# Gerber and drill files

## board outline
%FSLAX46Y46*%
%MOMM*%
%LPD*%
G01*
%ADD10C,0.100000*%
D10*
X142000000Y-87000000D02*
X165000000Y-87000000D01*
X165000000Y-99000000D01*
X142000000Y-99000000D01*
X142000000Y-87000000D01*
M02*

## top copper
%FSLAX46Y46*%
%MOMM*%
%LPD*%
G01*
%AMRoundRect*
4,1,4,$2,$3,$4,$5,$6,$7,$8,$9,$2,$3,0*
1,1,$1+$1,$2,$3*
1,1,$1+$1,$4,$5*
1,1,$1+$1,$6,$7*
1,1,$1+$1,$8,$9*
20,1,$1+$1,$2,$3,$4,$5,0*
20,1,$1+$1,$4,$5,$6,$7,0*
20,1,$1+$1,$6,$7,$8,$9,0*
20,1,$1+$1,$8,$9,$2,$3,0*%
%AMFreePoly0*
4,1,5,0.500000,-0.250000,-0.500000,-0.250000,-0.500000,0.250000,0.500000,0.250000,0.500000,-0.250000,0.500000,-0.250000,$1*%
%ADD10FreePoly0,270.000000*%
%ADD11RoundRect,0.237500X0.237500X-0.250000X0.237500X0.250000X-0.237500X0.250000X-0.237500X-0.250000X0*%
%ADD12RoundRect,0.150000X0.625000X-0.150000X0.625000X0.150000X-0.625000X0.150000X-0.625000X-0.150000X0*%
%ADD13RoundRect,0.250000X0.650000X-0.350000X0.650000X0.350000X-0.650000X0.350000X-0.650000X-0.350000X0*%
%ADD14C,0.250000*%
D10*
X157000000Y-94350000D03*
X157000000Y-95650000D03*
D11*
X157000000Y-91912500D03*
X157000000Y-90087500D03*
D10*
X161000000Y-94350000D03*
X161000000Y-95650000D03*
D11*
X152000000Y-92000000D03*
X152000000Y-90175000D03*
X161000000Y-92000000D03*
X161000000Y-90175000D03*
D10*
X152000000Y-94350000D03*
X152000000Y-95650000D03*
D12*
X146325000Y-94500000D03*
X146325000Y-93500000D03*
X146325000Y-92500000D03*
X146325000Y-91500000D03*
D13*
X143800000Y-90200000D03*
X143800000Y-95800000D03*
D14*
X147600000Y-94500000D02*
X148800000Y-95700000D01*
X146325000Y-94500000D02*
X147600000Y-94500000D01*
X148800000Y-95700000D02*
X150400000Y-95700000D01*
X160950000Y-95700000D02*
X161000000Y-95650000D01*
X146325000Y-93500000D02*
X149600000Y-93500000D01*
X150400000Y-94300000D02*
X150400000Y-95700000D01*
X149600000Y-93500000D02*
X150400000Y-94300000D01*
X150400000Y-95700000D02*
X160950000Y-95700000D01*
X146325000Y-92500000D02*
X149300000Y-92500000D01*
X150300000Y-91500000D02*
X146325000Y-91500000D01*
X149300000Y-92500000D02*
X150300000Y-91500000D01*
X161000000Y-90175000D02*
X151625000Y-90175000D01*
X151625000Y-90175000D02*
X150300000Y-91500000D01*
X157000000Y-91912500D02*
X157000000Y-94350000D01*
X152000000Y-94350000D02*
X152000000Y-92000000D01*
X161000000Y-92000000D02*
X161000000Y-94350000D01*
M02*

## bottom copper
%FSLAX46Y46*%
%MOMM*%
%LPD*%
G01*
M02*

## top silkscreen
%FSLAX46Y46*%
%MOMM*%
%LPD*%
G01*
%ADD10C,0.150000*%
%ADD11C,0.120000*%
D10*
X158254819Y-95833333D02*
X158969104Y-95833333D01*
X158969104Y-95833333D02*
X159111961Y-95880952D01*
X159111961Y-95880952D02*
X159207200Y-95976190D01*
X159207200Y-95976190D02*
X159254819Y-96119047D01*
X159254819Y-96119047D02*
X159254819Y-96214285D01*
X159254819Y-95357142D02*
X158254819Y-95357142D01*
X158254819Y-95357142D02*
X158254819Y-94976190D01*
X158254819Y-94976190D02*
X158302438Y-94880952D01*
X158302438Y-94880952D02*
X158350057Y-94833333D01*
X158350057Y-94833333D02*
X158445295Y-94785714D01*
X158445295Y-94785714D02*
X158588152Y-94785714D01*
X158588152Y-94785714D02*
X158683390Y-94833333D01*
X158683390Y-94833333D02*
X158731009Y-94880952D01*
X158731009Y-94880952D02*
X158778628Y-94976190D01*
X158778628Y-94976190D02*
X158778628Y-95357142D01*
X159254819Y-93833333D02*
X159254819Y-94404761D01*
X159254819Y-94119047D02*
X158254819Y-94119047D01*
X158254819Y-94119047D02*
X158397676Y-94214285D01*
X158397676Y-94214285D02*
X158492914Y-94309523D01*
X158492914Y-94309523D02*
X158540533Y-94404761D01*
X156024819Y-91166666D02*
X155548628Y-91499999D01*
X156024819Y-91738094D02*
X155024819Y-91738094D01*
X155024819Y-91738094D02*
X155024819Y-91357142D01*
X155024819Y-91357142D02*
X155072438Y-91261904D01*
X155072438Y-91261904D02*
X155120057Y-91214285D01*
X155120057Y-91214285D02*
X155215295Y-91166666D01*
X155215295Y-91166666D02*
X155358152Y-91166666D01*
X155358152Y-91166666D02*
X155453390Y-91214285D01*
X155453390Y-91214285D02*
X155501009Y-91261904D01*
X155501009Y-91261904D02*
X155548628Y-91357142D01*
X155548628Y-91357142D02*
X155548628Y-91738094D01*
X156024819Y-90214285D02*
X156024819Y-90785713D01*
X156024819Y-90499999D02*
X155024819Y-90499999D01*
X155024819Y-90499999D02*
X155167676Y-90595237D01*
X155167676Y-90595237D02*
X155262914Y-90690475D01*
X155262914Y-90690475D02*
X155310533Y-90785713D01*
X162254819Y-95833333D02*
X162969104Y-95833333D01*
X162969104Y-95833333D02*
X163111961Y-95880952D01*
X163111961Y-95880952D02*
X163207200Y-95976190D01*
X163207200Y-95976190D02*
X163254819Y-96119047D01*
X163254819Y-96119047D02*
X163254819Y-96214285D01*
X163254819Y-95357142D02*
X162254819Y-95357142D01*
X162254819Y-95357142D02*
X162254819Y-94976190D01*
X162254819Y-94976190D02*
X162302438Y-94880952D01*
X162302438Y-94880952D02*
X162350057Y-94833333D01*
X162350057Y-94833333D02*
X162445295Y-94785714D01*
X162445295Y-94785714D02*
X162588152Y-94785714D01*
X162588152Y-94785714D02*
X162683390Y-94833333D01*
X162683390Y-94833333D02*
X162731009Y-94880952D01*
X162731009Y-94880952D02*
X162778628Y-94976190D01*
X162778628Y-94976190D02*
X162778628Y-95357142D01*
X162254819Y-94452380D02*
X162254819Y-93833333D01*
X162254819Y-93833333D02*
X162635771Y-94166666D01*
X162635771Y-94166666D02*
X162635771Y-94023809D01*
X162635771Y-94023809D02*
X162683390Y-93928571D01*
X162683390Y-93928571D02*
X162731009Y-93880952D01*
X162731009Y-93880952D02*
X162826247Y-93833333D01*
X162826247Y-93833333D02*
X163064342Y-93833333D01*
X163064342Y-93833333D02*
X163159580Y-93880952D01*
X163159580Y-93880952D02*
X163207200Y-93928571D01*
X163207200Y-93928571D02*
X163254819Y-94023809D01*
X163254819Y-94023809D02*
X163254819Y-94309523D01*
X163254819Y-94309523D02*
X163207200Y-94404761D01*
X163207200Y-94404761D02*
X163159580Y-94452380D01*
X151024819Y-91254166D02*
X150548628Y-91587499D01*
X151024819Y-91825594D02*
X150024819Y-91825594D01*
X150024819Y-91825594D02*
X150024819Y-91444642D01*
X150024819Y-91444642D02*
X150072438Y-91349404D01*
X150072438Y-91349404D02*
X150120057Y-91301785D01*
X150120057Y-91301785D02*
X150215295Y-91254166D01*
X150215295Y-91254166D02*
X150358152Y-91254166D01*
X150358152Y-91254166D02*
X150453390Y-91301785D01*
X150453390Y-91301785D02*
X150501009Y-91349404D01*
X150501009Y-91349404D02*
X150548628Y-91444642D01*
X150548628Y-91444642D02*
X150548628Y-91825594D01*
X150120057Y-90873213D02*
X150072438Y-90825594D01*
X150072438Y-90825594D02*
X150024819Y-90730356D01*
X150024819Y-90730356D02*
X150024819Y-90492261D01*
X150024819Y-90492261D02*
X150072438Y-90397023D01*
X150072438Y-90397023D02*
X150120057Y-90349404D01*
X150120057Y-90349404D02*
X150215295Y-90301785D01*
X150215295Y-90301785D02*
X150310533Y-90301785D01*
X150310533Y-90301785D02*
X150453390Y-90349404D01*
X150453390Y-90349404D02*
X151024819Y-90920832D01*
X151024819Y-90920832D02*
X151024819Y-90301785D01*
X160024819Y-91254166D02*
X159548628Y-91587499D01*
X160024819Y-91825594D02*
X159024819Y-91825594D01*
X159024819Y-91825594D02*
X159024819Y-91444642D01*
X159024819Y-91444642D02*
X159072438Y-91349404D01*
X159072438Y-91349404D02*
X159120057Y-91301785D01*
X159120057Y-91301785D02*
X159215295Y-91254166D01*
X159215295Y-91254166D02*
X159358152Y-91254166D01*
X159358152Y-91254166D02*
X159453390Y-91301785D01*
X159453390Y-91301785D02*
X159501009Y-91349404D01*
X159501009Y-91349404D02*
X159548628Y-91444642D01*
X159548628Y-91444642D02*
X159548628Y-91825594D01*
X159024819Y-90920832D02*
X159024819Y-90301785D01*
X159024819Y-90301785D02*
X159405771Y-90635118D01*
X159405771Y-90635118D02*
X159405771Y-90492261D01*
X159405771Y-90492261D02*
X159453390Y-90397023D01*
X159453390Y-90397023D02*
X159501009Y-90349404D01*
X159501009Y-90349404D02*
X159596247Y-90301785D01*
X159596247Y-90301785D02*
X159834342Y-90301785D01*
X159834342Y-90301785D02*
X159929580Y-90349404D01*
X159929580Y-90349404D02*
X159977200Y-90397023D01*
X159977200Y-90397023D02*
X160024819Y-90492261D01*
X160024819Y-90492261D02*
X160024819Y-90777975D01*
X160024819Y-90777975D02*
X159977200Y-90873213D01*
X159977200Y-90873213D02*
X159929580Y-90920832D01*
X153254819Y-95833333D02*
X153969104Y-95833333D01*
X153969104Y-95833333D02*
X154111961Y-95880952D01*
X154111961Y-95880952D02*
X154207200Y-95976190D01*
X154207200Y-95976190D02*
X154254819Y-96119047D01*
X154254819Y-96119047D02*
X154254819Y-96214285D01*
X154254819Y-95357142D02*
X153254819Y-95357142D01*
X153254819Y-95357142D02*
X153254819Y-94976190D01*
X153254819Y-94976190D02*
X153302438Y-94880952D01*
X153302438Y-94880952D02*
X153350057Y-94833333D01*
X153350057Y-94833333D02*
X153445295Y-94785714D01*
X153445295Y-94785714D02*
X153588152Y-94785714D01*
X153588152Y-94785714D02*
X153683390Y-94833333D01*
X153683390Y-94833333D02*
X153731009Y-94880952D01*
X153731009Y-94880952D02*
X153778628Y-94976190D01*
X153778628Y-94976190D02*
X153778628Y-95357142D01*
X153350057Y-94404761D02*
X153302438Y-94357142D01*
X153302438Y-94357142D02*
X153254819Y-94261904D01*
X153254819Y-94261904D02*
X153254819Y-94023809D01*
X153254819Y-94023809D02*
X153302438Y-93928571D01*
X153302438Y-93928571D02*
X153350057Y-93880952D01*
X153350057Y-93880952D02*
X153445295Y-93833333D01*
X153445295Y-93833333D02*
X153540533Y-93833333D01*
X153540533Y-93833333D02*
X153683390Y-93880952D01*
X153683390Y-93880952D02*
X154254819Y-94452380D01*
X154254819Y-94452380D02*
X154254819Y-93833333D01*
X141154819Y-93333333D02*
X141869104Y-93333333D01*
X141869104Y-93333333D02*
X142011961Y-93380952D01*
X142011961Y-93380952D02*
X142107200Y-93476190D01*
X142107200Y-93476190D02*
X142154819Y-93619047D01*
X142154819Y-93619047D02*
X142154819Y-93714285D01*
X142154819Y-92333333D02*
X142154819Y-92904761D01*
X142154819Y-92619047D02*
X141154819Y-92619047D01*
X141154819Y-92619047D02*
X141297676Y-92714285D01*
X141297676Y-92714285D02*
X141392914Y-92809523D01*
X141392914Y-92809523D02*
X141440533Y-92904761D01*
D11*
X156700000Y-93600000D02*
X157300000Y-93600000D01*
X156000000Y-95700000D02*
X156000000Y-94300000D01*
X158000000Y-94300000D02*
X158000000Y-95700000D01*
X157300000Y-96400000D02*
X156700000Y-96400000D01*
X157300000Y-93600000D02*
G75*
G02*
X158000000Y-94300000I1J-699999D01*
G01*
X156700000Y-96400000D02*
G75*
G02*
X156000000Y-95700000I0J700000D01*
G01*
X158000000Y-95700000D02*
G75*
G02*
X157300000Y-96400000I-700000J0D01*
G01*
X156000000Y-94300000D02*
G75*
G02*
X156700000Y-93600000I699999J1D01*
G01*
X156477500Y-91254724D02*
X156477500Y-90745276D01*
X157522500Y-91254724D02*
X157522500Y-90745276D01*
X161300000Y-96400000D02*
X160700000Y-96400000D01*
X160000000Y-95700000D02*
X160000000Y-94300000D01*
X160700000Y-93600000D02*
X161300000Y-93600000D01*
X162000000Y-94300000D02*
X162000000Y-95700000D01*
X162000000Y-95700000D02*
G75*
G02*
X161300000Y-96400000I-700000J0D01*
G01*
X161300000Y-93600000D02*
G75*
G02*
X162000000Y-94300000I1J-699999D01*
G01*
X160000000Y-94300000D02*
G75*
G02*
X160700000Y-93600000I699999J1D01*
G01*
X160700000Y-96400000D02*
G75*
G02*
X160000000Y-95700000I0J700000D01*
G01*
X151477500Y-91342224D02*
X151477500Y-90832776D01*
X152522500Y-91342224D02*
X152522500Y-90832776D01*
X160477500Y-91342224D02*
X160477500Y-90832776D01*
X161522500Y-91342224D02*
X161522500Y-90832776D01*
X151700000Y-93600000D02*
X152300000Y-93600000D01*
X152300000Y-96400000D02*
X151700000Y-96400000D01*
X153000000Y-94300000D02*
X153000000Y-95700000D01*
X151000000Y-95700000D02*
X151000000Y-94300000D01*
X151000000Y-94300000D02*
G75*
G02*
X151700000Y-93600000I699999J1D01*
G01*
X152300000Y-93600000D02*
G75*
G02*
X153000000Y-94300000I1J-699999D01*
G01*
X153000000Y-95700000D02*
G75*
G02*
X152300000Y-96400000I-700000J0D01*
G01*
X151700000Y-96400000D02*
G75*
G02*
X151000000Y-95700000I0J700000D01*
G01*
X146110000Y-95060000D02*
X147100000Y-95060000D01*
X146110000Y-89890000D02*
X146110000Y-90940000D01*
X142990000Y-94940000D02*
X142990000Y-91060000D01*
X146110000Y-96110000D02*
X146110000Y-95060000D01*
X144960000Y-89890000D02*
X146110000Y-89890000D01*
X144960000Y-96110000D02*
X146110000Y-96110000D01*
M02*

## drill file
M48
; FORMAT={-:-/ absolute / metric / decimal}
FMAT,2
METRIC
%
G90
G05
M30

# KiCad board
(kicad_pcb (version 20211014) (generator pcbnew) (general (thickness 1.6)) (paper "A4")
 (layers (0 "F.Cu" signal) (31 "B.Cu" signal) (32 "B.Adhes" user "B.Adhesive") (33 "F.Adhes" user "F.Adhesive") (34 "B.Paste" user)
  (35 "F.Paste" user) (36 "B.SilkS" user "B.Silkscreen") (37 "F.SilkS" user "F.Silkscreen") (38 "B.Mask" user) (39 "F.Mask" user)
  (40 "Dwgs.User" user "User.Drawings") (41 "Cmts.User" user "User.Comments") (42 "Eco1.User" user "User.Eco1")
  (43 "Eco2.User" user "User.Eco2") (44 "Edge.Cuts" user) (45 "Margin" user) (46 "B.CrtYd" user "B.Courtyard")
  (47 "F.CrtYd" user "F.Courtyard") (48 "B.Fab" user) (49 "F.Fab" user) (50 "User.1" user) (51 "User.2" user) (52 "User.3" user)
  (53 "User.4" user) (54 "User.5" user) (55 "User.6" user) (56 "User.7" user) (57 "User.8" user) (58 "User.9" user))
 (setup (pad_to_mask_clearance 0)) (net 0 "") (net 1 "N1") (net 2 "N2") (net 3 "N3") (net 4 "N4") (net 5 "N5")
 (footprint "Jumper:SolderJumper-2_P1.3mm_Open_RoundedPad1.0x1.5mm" (layer "F.Cu") (at 157 95 -90)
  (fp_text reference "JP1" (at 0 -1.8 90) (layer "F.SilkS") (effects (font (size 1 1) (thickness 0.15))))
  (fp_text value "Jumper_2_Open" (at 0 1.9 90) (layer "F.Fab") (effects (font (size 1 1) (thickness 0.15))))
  (fp_line (start -1.4 0.3) (end -1.4 -0.3) (layer "F.SilkS") (width 0.12))
  (fp_line (start 0.7 1) (end -0.7 1) (layer "F.SilkS") (width 0.12))
  (fp_line (start -0.7 -1) (end 0.7 -1) (layer "F.SilkS") (width 0.12))
  (fp_line (start 1.4 -0.3) (end 1.4 0.3) (layer "F.SilkS") (width 0.12))
  (fp_arc (start -1.4 -0.3) (mid -1.194975 -0.794975) (end -0.7 -1) (layer "F.SilkS") (width 0.12))
  (fp_arc (start 1.4 0.3) (mid 1.194975 0.794975) (end 0.7 1) (layer "F.SilkS") (width 0.12))
  (fp_arc (start 0.7 -1) (mid 1.194975 -0.794975) (end 1.4 -0.3) (layer "F.SilkS") (width 0.12))
  (fp_arc (start -0.7 1) (mid -1.194975 0.794975) (end -1.4 0.3) (layer "F.SilkS") (width 0.12))
  (pad "1" smd custom (at -0.65 0 270) (size 1 0.5) (layers "F.Cu" "F.Mask") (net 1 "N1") (zone_connect 2)
   (options (clearance outline) (anchor rect)) (primitives))
  (pad "2" smd custom (at 0.65 0 270) (size 1 0.5) (layers "F.Cu" "F.Mask") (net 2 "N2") (zone_connect 2)
   (options (clearance outline) (anchor rect)) (primitives)))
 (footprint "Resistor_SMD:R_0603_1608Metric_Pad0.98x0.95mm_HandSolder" (layer "F.Cu") (at 157 91 90)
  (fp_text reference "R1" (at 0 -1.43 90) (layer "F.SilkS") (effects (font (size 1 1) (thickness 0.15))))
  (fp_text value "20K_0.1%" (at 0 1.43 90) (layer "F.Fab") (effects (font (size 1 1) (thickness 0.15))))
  (fp_line (start -0.254724 -0.5225) (end 0.254724 -0.5225) (layer "F.SilkS") (width 0.12))
  (fp_line (start -0.254724 0.5225) (end 0.254724 0.5225) (layer "F.SilkS") (width 0.12))
  (pad "1" smd roundrect (at -0.9125 0 90) (size 0.975 0.95) (layers "F.Cu" "F.Paste" "F.Mask") (roundrect_rratio 0.25) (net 1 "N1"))
  (pad "2" smd roundrect (at 0.9125 0 90) (size 0.975 0.95) (layers "F.Cu" "F.Paste" "F.Mask") (roundrect_rratio 0.25) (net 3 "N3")))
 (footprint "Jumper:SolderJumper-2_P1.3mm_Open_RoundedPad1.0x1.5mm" (layer "F.Cu") (at 161 95 -90)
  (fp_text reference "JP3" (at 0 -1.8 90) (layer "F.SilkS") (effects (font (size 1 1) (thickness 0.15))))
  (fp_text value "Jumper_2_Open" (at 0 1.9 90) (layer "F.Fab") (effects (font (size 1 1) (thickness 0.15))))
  (fp_line (start 1.4 -0.3) (end 1.4 0.3) (layer "F.SilkS") (width 0.12))
  (fp_line (start 0.7 1) (end -0.7 1) (layer "F.SilkS") (width 0.12))
  (fp_line (start -1.4 0.3) (end -1.4 -0.3) (layer "F.SilkS") (width 0.12))
  (fp_line (start -0.7 -1) (end 0.7 -1) (layer "F.SilkS") (width 0.12))
  (fp_arc (start 0.7 -1) (mid 1.194975 -0.794975) (end 1.4 -0.3) (layer "F.SilkS") (width 0.12))
  (fp_arc (start -1.4 -0.3) (mid -1.194975 -0.794975) (end -0.7 -1) (layer "F.SilkS") (width 0.12))
  (fp_arc (start -0.7 1) (mid -1.194975 0.794975) (end -1.4 0.3) (layer "F.SilkS") (width 0.12))
  (fp_arc (start 1.4 0.3) (mid 1.194975 0.794975) (end 0.7 1) (layer "F.SilkS") (width 0.12))
  (pad "1" smd custom (at -0.65 0 270) (size 1 0.5) (layers "F.Cu" "F.Mask") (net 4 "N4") (zone_connect 2)
   (options (clearance outline) (anchor rect)) (primitives))
  (pad "2" smd custom (at 0.65 0 270) (size 1 0.5) (layers "F.Cu" "F.Mask") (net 2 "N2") (zone_connect 2)
   (options (clearance outline) (anchor rect)) (primitives)))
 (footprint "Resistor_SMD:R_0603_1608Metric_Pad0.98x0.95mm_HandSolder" (layer "F.Cu") (at 152 91.0875 90)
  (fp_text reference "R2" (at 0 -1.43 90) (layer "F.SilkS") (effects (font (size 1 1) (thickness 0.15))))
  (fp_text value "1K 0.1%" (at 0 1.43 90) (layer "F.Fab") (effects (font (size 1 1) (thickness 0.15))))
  (fp_line (start -0.254724 -0.5225) (end 0.254724 -0.5225) (layer "F.SilkS") (width 0.12))
  (fp_line (start -0.254724 0.5225) (end 0.254724 0.5225) (layer "F.SilkS") (width 0.12))
  (pad "1" smd roundrect (at -0.9125 0 90) (size 0.975 0.95) (layers "F.Cu" "F.Paste" "F.Mask") (roundrect_rratio 0.25) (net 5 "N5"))
  (pad "2" smd roundrect (at 0.9125 0 90) (size 0.975 0.95) (layers "F.Cu" "F.Paste" "F.Mask") (roundrect_rratio 0.25) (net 3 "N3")))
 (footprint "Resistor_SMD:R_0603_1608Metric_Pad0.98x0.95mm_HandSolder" (layer "F.Cu") (at 161 91.0875 90)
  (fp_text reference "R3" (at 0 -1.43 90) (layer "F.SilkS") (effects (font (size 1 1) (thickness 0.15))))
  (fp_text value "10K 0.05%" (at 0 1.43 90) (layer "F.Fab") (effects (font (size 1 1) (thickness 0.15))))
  (fp_line (start -0.254724 -0.5225) (end 0.254724 -0.5225) (layer "F.SilkS") (width 0.12))
  (fp_line (start -0.254724 0.5225) (end 0.254724 0.5225) (layer "F.SilkS") (width 0.12))
  (pad "1" smd roundrect (at -0.9125 0 90) (size 0.975 0.95) (layers "F.Cu" "F.Paste" "F.Mask") (roundrect_rratio 0.25) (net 4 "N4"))
  (pad "2" smd roundrect (at 0.9125 0 90) (size 0.975 0.95) (layers "F.Cu" "F.Paste" "F.Mask") (roundrect_rratio 0.25) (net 3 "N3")))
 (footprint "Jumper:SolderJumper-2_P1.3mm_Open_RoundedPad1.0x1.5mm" (layer "F.Cu") (at 152 95 -90)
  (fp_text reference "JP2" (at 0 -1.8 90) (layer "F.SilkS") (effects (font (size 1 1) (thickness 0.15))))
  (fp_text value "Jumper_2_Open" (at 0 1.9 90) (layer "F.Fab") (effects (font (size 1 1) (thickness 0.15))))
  (fp_line (start -1.4 0.3) (end -1.4 -0.3) (layer "F.SilkS") (width 0.12))
  (fp_line (start 1.4 -0.3) (end 1.4 0.3) (layer "F.SilkS") (width 0.12))
  (fp_line (start -0.7 -1) (end 0.7 -1) (layer "F.SilkS") (width 0.12))
  (fp_line (start 0.7 1) (end -0.7 1) (layer "F.SilkS") (width 0.12))
  (fp_arc (start -0.7 1) (mid -1.194975 0.794975) (end -1.4 0.3) (layer "F.SilkS") (width 0.12))
  (fp_arc (start -1.4 -0.3) (mid -1.194975 -0.794975) (end -0.7 -1) (layer "F.SilkS") (width 0.12))
  (fp_arc (start 0.7 -1) (mid 1.194975 -0.794975) (end 1.4 -0.3) (layer "F.SilkS") (width 0.12))
  (fp_arc (start 1.4 0.3) (mid 1.194975 0.794975) (end 0.7 1) (layer "F.SilkS") (width 0.12))
  (pad "1" smd custom (at -0.65 0 270) (size 1 0.5) (layers "F.Cu" "F.Mask") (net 5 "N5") (zone_connect 2)
   (options (clearance outline) (anchor rect)) (primitives))
  (pad "2" smd custom (at 0.65 0 270) (size 1 0.5) (layers "F.Cu" "F.Mask") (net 2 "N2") (zone_connect 2)
   (options (clearance outline) (anchor rect)) (primitives)))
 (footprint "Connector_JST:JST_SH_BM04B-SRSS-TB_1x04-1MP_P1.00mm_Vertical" (layer "F.Cu") (at 145 93 90)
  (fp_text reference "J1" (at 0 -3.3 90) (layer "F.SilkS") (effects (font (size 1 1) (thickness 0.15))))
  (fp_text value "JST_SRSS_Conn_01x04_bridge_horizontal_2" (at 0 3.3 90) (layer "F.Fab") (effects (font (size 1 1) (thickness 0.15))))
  (fp_line (start -2.06 1.11) (end -2.06 2.1) (layer "F.SilkS") (width 0.12))
  (fp_line (start 3.11 1.11) (end 2.06 1.11) (layer "F.SilkS") (width 0.12))
  (fp_line (start -1.94 -2.01) (end 1.94 -2.01) (layer "F.SilkS") (width 0.12))
  (fp_line (start -3.11 1.11) (end -2.06 1.11) (layer "F.SilkS") (width 0.12))
  (fp_line (start 3.11 -0.04) (end 3.11 1.11) (layer "F.SilkS") (width 0.12))
  (fp_line (start -3.11 -0.04) (end -3.11 1.11) (layer "F.SilkS") (width 0.12))
  (pad "1" smd roundrect (at -1.5 1.325 90) (size 0.6 1.55) (layers "F.Cu" "F.Paste" "F.Mask") (roundrect_rratio 0.25) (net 2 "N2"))
  (pad "2" smd roundrect (at -0.5 1.325 90) (size 0.6 1.55) (layers "F.Cu" "F.Paste" "F.Mask") (roundrect_rratio 0.25) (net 2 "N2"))
  (pad "3" smd roundrect (at 0.5 1.325 90) (size 0.6 1.55) (layers "F.Cu" "F.Paste" "F.Mask") (roundrect_rratio 0.25) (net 3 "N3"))
  (pad "4" smd roundrect (at 1.5 1.325 90) (size 0.6 1.55) (layers "F.Cu" "F.Paste" "F.Mask") (roundrect_rratio 0.25) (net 3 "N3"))
  (pad "MP" smd roundrect (at 2.8 -1.2 90) (size 1.2 1.8) (layers "F.Cu" "F.Paste" "F.Mask") (roundrect_rratio 0.2083333333))
  (pad "MP" smd roundrect (at -2.8 -1.2 90) (size 1.2 1.8) (layers "F.Cu" "F.Paste" "F.Mask") (roundrect_rratio 0.2083333333)))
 (gr_rect (start 142 87) (end 165 99) (layer "Edge.Cuts") (width 0.1) (fill none))
 (segment (start 147.6 94.5) (end 148.8 95.7) (width 0.25) (layer "F.Cu") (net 2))
 (segment (start 146.325 94.5) (end 147.6 94.5) (width 0.25) (layer "F.Cu") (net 2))
 (segment (start 148.8 95.7) (end 150.4 95.7) (width 0.25) (layer "F.Cu") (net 2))
 (segment (start 160.95 95.7) (end 161 95.65) (width 0.25) (layer "F.Cu") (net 2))
 (segment (start 146.325 93.5) (end 149.6 93.5) (width 0.25) (layer "F.Cu") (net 2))
 (segment (start 150.4 94.3) (end 150.4 95.7) (width 0.25) (layer "F.Cu") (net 2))
 (segment (start 149.6 93.5) (end 150.4 94.3) (width 0.25) (layer "F.Cu") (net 2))
 (segment (start 150.4 95.7) (end 160.95 95.7) (width 0.25) (layer "F.Cu") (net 2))
 (segment (start 146.325 92.5) (end 149.3 92.5) (width 0.25) (layer "F.Cu") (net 3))
 (segment (start 150.3 91.5) (end 146.325 91.5) (width 0.25) (layer "F.Cu") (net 3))
 (segment (start 149.3 92.5) (end 150.3 91.5) (width 0.25) (layer "F.Cu") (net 3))
 (segment (start 161 90.175) (end 151.625 90.175) (width 0.25) (layer "F.Cu") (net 3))
 (segment (start 151.625 90.175) (end 150.3 91.5) (width 0.25) (layer "F.Cu") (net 3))
 (segment (start 157 91.9125) (end 157 94.35) (width 0.25) (layer "F.Cu") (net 1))
 (segment (start 152 94.35) (end 152 92) (width 0.25) (layer "F.Cu") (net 5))
 (segment (start 161 92) (end 161 94.35) (width 0.25) (layer "F.Cu") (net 4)))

